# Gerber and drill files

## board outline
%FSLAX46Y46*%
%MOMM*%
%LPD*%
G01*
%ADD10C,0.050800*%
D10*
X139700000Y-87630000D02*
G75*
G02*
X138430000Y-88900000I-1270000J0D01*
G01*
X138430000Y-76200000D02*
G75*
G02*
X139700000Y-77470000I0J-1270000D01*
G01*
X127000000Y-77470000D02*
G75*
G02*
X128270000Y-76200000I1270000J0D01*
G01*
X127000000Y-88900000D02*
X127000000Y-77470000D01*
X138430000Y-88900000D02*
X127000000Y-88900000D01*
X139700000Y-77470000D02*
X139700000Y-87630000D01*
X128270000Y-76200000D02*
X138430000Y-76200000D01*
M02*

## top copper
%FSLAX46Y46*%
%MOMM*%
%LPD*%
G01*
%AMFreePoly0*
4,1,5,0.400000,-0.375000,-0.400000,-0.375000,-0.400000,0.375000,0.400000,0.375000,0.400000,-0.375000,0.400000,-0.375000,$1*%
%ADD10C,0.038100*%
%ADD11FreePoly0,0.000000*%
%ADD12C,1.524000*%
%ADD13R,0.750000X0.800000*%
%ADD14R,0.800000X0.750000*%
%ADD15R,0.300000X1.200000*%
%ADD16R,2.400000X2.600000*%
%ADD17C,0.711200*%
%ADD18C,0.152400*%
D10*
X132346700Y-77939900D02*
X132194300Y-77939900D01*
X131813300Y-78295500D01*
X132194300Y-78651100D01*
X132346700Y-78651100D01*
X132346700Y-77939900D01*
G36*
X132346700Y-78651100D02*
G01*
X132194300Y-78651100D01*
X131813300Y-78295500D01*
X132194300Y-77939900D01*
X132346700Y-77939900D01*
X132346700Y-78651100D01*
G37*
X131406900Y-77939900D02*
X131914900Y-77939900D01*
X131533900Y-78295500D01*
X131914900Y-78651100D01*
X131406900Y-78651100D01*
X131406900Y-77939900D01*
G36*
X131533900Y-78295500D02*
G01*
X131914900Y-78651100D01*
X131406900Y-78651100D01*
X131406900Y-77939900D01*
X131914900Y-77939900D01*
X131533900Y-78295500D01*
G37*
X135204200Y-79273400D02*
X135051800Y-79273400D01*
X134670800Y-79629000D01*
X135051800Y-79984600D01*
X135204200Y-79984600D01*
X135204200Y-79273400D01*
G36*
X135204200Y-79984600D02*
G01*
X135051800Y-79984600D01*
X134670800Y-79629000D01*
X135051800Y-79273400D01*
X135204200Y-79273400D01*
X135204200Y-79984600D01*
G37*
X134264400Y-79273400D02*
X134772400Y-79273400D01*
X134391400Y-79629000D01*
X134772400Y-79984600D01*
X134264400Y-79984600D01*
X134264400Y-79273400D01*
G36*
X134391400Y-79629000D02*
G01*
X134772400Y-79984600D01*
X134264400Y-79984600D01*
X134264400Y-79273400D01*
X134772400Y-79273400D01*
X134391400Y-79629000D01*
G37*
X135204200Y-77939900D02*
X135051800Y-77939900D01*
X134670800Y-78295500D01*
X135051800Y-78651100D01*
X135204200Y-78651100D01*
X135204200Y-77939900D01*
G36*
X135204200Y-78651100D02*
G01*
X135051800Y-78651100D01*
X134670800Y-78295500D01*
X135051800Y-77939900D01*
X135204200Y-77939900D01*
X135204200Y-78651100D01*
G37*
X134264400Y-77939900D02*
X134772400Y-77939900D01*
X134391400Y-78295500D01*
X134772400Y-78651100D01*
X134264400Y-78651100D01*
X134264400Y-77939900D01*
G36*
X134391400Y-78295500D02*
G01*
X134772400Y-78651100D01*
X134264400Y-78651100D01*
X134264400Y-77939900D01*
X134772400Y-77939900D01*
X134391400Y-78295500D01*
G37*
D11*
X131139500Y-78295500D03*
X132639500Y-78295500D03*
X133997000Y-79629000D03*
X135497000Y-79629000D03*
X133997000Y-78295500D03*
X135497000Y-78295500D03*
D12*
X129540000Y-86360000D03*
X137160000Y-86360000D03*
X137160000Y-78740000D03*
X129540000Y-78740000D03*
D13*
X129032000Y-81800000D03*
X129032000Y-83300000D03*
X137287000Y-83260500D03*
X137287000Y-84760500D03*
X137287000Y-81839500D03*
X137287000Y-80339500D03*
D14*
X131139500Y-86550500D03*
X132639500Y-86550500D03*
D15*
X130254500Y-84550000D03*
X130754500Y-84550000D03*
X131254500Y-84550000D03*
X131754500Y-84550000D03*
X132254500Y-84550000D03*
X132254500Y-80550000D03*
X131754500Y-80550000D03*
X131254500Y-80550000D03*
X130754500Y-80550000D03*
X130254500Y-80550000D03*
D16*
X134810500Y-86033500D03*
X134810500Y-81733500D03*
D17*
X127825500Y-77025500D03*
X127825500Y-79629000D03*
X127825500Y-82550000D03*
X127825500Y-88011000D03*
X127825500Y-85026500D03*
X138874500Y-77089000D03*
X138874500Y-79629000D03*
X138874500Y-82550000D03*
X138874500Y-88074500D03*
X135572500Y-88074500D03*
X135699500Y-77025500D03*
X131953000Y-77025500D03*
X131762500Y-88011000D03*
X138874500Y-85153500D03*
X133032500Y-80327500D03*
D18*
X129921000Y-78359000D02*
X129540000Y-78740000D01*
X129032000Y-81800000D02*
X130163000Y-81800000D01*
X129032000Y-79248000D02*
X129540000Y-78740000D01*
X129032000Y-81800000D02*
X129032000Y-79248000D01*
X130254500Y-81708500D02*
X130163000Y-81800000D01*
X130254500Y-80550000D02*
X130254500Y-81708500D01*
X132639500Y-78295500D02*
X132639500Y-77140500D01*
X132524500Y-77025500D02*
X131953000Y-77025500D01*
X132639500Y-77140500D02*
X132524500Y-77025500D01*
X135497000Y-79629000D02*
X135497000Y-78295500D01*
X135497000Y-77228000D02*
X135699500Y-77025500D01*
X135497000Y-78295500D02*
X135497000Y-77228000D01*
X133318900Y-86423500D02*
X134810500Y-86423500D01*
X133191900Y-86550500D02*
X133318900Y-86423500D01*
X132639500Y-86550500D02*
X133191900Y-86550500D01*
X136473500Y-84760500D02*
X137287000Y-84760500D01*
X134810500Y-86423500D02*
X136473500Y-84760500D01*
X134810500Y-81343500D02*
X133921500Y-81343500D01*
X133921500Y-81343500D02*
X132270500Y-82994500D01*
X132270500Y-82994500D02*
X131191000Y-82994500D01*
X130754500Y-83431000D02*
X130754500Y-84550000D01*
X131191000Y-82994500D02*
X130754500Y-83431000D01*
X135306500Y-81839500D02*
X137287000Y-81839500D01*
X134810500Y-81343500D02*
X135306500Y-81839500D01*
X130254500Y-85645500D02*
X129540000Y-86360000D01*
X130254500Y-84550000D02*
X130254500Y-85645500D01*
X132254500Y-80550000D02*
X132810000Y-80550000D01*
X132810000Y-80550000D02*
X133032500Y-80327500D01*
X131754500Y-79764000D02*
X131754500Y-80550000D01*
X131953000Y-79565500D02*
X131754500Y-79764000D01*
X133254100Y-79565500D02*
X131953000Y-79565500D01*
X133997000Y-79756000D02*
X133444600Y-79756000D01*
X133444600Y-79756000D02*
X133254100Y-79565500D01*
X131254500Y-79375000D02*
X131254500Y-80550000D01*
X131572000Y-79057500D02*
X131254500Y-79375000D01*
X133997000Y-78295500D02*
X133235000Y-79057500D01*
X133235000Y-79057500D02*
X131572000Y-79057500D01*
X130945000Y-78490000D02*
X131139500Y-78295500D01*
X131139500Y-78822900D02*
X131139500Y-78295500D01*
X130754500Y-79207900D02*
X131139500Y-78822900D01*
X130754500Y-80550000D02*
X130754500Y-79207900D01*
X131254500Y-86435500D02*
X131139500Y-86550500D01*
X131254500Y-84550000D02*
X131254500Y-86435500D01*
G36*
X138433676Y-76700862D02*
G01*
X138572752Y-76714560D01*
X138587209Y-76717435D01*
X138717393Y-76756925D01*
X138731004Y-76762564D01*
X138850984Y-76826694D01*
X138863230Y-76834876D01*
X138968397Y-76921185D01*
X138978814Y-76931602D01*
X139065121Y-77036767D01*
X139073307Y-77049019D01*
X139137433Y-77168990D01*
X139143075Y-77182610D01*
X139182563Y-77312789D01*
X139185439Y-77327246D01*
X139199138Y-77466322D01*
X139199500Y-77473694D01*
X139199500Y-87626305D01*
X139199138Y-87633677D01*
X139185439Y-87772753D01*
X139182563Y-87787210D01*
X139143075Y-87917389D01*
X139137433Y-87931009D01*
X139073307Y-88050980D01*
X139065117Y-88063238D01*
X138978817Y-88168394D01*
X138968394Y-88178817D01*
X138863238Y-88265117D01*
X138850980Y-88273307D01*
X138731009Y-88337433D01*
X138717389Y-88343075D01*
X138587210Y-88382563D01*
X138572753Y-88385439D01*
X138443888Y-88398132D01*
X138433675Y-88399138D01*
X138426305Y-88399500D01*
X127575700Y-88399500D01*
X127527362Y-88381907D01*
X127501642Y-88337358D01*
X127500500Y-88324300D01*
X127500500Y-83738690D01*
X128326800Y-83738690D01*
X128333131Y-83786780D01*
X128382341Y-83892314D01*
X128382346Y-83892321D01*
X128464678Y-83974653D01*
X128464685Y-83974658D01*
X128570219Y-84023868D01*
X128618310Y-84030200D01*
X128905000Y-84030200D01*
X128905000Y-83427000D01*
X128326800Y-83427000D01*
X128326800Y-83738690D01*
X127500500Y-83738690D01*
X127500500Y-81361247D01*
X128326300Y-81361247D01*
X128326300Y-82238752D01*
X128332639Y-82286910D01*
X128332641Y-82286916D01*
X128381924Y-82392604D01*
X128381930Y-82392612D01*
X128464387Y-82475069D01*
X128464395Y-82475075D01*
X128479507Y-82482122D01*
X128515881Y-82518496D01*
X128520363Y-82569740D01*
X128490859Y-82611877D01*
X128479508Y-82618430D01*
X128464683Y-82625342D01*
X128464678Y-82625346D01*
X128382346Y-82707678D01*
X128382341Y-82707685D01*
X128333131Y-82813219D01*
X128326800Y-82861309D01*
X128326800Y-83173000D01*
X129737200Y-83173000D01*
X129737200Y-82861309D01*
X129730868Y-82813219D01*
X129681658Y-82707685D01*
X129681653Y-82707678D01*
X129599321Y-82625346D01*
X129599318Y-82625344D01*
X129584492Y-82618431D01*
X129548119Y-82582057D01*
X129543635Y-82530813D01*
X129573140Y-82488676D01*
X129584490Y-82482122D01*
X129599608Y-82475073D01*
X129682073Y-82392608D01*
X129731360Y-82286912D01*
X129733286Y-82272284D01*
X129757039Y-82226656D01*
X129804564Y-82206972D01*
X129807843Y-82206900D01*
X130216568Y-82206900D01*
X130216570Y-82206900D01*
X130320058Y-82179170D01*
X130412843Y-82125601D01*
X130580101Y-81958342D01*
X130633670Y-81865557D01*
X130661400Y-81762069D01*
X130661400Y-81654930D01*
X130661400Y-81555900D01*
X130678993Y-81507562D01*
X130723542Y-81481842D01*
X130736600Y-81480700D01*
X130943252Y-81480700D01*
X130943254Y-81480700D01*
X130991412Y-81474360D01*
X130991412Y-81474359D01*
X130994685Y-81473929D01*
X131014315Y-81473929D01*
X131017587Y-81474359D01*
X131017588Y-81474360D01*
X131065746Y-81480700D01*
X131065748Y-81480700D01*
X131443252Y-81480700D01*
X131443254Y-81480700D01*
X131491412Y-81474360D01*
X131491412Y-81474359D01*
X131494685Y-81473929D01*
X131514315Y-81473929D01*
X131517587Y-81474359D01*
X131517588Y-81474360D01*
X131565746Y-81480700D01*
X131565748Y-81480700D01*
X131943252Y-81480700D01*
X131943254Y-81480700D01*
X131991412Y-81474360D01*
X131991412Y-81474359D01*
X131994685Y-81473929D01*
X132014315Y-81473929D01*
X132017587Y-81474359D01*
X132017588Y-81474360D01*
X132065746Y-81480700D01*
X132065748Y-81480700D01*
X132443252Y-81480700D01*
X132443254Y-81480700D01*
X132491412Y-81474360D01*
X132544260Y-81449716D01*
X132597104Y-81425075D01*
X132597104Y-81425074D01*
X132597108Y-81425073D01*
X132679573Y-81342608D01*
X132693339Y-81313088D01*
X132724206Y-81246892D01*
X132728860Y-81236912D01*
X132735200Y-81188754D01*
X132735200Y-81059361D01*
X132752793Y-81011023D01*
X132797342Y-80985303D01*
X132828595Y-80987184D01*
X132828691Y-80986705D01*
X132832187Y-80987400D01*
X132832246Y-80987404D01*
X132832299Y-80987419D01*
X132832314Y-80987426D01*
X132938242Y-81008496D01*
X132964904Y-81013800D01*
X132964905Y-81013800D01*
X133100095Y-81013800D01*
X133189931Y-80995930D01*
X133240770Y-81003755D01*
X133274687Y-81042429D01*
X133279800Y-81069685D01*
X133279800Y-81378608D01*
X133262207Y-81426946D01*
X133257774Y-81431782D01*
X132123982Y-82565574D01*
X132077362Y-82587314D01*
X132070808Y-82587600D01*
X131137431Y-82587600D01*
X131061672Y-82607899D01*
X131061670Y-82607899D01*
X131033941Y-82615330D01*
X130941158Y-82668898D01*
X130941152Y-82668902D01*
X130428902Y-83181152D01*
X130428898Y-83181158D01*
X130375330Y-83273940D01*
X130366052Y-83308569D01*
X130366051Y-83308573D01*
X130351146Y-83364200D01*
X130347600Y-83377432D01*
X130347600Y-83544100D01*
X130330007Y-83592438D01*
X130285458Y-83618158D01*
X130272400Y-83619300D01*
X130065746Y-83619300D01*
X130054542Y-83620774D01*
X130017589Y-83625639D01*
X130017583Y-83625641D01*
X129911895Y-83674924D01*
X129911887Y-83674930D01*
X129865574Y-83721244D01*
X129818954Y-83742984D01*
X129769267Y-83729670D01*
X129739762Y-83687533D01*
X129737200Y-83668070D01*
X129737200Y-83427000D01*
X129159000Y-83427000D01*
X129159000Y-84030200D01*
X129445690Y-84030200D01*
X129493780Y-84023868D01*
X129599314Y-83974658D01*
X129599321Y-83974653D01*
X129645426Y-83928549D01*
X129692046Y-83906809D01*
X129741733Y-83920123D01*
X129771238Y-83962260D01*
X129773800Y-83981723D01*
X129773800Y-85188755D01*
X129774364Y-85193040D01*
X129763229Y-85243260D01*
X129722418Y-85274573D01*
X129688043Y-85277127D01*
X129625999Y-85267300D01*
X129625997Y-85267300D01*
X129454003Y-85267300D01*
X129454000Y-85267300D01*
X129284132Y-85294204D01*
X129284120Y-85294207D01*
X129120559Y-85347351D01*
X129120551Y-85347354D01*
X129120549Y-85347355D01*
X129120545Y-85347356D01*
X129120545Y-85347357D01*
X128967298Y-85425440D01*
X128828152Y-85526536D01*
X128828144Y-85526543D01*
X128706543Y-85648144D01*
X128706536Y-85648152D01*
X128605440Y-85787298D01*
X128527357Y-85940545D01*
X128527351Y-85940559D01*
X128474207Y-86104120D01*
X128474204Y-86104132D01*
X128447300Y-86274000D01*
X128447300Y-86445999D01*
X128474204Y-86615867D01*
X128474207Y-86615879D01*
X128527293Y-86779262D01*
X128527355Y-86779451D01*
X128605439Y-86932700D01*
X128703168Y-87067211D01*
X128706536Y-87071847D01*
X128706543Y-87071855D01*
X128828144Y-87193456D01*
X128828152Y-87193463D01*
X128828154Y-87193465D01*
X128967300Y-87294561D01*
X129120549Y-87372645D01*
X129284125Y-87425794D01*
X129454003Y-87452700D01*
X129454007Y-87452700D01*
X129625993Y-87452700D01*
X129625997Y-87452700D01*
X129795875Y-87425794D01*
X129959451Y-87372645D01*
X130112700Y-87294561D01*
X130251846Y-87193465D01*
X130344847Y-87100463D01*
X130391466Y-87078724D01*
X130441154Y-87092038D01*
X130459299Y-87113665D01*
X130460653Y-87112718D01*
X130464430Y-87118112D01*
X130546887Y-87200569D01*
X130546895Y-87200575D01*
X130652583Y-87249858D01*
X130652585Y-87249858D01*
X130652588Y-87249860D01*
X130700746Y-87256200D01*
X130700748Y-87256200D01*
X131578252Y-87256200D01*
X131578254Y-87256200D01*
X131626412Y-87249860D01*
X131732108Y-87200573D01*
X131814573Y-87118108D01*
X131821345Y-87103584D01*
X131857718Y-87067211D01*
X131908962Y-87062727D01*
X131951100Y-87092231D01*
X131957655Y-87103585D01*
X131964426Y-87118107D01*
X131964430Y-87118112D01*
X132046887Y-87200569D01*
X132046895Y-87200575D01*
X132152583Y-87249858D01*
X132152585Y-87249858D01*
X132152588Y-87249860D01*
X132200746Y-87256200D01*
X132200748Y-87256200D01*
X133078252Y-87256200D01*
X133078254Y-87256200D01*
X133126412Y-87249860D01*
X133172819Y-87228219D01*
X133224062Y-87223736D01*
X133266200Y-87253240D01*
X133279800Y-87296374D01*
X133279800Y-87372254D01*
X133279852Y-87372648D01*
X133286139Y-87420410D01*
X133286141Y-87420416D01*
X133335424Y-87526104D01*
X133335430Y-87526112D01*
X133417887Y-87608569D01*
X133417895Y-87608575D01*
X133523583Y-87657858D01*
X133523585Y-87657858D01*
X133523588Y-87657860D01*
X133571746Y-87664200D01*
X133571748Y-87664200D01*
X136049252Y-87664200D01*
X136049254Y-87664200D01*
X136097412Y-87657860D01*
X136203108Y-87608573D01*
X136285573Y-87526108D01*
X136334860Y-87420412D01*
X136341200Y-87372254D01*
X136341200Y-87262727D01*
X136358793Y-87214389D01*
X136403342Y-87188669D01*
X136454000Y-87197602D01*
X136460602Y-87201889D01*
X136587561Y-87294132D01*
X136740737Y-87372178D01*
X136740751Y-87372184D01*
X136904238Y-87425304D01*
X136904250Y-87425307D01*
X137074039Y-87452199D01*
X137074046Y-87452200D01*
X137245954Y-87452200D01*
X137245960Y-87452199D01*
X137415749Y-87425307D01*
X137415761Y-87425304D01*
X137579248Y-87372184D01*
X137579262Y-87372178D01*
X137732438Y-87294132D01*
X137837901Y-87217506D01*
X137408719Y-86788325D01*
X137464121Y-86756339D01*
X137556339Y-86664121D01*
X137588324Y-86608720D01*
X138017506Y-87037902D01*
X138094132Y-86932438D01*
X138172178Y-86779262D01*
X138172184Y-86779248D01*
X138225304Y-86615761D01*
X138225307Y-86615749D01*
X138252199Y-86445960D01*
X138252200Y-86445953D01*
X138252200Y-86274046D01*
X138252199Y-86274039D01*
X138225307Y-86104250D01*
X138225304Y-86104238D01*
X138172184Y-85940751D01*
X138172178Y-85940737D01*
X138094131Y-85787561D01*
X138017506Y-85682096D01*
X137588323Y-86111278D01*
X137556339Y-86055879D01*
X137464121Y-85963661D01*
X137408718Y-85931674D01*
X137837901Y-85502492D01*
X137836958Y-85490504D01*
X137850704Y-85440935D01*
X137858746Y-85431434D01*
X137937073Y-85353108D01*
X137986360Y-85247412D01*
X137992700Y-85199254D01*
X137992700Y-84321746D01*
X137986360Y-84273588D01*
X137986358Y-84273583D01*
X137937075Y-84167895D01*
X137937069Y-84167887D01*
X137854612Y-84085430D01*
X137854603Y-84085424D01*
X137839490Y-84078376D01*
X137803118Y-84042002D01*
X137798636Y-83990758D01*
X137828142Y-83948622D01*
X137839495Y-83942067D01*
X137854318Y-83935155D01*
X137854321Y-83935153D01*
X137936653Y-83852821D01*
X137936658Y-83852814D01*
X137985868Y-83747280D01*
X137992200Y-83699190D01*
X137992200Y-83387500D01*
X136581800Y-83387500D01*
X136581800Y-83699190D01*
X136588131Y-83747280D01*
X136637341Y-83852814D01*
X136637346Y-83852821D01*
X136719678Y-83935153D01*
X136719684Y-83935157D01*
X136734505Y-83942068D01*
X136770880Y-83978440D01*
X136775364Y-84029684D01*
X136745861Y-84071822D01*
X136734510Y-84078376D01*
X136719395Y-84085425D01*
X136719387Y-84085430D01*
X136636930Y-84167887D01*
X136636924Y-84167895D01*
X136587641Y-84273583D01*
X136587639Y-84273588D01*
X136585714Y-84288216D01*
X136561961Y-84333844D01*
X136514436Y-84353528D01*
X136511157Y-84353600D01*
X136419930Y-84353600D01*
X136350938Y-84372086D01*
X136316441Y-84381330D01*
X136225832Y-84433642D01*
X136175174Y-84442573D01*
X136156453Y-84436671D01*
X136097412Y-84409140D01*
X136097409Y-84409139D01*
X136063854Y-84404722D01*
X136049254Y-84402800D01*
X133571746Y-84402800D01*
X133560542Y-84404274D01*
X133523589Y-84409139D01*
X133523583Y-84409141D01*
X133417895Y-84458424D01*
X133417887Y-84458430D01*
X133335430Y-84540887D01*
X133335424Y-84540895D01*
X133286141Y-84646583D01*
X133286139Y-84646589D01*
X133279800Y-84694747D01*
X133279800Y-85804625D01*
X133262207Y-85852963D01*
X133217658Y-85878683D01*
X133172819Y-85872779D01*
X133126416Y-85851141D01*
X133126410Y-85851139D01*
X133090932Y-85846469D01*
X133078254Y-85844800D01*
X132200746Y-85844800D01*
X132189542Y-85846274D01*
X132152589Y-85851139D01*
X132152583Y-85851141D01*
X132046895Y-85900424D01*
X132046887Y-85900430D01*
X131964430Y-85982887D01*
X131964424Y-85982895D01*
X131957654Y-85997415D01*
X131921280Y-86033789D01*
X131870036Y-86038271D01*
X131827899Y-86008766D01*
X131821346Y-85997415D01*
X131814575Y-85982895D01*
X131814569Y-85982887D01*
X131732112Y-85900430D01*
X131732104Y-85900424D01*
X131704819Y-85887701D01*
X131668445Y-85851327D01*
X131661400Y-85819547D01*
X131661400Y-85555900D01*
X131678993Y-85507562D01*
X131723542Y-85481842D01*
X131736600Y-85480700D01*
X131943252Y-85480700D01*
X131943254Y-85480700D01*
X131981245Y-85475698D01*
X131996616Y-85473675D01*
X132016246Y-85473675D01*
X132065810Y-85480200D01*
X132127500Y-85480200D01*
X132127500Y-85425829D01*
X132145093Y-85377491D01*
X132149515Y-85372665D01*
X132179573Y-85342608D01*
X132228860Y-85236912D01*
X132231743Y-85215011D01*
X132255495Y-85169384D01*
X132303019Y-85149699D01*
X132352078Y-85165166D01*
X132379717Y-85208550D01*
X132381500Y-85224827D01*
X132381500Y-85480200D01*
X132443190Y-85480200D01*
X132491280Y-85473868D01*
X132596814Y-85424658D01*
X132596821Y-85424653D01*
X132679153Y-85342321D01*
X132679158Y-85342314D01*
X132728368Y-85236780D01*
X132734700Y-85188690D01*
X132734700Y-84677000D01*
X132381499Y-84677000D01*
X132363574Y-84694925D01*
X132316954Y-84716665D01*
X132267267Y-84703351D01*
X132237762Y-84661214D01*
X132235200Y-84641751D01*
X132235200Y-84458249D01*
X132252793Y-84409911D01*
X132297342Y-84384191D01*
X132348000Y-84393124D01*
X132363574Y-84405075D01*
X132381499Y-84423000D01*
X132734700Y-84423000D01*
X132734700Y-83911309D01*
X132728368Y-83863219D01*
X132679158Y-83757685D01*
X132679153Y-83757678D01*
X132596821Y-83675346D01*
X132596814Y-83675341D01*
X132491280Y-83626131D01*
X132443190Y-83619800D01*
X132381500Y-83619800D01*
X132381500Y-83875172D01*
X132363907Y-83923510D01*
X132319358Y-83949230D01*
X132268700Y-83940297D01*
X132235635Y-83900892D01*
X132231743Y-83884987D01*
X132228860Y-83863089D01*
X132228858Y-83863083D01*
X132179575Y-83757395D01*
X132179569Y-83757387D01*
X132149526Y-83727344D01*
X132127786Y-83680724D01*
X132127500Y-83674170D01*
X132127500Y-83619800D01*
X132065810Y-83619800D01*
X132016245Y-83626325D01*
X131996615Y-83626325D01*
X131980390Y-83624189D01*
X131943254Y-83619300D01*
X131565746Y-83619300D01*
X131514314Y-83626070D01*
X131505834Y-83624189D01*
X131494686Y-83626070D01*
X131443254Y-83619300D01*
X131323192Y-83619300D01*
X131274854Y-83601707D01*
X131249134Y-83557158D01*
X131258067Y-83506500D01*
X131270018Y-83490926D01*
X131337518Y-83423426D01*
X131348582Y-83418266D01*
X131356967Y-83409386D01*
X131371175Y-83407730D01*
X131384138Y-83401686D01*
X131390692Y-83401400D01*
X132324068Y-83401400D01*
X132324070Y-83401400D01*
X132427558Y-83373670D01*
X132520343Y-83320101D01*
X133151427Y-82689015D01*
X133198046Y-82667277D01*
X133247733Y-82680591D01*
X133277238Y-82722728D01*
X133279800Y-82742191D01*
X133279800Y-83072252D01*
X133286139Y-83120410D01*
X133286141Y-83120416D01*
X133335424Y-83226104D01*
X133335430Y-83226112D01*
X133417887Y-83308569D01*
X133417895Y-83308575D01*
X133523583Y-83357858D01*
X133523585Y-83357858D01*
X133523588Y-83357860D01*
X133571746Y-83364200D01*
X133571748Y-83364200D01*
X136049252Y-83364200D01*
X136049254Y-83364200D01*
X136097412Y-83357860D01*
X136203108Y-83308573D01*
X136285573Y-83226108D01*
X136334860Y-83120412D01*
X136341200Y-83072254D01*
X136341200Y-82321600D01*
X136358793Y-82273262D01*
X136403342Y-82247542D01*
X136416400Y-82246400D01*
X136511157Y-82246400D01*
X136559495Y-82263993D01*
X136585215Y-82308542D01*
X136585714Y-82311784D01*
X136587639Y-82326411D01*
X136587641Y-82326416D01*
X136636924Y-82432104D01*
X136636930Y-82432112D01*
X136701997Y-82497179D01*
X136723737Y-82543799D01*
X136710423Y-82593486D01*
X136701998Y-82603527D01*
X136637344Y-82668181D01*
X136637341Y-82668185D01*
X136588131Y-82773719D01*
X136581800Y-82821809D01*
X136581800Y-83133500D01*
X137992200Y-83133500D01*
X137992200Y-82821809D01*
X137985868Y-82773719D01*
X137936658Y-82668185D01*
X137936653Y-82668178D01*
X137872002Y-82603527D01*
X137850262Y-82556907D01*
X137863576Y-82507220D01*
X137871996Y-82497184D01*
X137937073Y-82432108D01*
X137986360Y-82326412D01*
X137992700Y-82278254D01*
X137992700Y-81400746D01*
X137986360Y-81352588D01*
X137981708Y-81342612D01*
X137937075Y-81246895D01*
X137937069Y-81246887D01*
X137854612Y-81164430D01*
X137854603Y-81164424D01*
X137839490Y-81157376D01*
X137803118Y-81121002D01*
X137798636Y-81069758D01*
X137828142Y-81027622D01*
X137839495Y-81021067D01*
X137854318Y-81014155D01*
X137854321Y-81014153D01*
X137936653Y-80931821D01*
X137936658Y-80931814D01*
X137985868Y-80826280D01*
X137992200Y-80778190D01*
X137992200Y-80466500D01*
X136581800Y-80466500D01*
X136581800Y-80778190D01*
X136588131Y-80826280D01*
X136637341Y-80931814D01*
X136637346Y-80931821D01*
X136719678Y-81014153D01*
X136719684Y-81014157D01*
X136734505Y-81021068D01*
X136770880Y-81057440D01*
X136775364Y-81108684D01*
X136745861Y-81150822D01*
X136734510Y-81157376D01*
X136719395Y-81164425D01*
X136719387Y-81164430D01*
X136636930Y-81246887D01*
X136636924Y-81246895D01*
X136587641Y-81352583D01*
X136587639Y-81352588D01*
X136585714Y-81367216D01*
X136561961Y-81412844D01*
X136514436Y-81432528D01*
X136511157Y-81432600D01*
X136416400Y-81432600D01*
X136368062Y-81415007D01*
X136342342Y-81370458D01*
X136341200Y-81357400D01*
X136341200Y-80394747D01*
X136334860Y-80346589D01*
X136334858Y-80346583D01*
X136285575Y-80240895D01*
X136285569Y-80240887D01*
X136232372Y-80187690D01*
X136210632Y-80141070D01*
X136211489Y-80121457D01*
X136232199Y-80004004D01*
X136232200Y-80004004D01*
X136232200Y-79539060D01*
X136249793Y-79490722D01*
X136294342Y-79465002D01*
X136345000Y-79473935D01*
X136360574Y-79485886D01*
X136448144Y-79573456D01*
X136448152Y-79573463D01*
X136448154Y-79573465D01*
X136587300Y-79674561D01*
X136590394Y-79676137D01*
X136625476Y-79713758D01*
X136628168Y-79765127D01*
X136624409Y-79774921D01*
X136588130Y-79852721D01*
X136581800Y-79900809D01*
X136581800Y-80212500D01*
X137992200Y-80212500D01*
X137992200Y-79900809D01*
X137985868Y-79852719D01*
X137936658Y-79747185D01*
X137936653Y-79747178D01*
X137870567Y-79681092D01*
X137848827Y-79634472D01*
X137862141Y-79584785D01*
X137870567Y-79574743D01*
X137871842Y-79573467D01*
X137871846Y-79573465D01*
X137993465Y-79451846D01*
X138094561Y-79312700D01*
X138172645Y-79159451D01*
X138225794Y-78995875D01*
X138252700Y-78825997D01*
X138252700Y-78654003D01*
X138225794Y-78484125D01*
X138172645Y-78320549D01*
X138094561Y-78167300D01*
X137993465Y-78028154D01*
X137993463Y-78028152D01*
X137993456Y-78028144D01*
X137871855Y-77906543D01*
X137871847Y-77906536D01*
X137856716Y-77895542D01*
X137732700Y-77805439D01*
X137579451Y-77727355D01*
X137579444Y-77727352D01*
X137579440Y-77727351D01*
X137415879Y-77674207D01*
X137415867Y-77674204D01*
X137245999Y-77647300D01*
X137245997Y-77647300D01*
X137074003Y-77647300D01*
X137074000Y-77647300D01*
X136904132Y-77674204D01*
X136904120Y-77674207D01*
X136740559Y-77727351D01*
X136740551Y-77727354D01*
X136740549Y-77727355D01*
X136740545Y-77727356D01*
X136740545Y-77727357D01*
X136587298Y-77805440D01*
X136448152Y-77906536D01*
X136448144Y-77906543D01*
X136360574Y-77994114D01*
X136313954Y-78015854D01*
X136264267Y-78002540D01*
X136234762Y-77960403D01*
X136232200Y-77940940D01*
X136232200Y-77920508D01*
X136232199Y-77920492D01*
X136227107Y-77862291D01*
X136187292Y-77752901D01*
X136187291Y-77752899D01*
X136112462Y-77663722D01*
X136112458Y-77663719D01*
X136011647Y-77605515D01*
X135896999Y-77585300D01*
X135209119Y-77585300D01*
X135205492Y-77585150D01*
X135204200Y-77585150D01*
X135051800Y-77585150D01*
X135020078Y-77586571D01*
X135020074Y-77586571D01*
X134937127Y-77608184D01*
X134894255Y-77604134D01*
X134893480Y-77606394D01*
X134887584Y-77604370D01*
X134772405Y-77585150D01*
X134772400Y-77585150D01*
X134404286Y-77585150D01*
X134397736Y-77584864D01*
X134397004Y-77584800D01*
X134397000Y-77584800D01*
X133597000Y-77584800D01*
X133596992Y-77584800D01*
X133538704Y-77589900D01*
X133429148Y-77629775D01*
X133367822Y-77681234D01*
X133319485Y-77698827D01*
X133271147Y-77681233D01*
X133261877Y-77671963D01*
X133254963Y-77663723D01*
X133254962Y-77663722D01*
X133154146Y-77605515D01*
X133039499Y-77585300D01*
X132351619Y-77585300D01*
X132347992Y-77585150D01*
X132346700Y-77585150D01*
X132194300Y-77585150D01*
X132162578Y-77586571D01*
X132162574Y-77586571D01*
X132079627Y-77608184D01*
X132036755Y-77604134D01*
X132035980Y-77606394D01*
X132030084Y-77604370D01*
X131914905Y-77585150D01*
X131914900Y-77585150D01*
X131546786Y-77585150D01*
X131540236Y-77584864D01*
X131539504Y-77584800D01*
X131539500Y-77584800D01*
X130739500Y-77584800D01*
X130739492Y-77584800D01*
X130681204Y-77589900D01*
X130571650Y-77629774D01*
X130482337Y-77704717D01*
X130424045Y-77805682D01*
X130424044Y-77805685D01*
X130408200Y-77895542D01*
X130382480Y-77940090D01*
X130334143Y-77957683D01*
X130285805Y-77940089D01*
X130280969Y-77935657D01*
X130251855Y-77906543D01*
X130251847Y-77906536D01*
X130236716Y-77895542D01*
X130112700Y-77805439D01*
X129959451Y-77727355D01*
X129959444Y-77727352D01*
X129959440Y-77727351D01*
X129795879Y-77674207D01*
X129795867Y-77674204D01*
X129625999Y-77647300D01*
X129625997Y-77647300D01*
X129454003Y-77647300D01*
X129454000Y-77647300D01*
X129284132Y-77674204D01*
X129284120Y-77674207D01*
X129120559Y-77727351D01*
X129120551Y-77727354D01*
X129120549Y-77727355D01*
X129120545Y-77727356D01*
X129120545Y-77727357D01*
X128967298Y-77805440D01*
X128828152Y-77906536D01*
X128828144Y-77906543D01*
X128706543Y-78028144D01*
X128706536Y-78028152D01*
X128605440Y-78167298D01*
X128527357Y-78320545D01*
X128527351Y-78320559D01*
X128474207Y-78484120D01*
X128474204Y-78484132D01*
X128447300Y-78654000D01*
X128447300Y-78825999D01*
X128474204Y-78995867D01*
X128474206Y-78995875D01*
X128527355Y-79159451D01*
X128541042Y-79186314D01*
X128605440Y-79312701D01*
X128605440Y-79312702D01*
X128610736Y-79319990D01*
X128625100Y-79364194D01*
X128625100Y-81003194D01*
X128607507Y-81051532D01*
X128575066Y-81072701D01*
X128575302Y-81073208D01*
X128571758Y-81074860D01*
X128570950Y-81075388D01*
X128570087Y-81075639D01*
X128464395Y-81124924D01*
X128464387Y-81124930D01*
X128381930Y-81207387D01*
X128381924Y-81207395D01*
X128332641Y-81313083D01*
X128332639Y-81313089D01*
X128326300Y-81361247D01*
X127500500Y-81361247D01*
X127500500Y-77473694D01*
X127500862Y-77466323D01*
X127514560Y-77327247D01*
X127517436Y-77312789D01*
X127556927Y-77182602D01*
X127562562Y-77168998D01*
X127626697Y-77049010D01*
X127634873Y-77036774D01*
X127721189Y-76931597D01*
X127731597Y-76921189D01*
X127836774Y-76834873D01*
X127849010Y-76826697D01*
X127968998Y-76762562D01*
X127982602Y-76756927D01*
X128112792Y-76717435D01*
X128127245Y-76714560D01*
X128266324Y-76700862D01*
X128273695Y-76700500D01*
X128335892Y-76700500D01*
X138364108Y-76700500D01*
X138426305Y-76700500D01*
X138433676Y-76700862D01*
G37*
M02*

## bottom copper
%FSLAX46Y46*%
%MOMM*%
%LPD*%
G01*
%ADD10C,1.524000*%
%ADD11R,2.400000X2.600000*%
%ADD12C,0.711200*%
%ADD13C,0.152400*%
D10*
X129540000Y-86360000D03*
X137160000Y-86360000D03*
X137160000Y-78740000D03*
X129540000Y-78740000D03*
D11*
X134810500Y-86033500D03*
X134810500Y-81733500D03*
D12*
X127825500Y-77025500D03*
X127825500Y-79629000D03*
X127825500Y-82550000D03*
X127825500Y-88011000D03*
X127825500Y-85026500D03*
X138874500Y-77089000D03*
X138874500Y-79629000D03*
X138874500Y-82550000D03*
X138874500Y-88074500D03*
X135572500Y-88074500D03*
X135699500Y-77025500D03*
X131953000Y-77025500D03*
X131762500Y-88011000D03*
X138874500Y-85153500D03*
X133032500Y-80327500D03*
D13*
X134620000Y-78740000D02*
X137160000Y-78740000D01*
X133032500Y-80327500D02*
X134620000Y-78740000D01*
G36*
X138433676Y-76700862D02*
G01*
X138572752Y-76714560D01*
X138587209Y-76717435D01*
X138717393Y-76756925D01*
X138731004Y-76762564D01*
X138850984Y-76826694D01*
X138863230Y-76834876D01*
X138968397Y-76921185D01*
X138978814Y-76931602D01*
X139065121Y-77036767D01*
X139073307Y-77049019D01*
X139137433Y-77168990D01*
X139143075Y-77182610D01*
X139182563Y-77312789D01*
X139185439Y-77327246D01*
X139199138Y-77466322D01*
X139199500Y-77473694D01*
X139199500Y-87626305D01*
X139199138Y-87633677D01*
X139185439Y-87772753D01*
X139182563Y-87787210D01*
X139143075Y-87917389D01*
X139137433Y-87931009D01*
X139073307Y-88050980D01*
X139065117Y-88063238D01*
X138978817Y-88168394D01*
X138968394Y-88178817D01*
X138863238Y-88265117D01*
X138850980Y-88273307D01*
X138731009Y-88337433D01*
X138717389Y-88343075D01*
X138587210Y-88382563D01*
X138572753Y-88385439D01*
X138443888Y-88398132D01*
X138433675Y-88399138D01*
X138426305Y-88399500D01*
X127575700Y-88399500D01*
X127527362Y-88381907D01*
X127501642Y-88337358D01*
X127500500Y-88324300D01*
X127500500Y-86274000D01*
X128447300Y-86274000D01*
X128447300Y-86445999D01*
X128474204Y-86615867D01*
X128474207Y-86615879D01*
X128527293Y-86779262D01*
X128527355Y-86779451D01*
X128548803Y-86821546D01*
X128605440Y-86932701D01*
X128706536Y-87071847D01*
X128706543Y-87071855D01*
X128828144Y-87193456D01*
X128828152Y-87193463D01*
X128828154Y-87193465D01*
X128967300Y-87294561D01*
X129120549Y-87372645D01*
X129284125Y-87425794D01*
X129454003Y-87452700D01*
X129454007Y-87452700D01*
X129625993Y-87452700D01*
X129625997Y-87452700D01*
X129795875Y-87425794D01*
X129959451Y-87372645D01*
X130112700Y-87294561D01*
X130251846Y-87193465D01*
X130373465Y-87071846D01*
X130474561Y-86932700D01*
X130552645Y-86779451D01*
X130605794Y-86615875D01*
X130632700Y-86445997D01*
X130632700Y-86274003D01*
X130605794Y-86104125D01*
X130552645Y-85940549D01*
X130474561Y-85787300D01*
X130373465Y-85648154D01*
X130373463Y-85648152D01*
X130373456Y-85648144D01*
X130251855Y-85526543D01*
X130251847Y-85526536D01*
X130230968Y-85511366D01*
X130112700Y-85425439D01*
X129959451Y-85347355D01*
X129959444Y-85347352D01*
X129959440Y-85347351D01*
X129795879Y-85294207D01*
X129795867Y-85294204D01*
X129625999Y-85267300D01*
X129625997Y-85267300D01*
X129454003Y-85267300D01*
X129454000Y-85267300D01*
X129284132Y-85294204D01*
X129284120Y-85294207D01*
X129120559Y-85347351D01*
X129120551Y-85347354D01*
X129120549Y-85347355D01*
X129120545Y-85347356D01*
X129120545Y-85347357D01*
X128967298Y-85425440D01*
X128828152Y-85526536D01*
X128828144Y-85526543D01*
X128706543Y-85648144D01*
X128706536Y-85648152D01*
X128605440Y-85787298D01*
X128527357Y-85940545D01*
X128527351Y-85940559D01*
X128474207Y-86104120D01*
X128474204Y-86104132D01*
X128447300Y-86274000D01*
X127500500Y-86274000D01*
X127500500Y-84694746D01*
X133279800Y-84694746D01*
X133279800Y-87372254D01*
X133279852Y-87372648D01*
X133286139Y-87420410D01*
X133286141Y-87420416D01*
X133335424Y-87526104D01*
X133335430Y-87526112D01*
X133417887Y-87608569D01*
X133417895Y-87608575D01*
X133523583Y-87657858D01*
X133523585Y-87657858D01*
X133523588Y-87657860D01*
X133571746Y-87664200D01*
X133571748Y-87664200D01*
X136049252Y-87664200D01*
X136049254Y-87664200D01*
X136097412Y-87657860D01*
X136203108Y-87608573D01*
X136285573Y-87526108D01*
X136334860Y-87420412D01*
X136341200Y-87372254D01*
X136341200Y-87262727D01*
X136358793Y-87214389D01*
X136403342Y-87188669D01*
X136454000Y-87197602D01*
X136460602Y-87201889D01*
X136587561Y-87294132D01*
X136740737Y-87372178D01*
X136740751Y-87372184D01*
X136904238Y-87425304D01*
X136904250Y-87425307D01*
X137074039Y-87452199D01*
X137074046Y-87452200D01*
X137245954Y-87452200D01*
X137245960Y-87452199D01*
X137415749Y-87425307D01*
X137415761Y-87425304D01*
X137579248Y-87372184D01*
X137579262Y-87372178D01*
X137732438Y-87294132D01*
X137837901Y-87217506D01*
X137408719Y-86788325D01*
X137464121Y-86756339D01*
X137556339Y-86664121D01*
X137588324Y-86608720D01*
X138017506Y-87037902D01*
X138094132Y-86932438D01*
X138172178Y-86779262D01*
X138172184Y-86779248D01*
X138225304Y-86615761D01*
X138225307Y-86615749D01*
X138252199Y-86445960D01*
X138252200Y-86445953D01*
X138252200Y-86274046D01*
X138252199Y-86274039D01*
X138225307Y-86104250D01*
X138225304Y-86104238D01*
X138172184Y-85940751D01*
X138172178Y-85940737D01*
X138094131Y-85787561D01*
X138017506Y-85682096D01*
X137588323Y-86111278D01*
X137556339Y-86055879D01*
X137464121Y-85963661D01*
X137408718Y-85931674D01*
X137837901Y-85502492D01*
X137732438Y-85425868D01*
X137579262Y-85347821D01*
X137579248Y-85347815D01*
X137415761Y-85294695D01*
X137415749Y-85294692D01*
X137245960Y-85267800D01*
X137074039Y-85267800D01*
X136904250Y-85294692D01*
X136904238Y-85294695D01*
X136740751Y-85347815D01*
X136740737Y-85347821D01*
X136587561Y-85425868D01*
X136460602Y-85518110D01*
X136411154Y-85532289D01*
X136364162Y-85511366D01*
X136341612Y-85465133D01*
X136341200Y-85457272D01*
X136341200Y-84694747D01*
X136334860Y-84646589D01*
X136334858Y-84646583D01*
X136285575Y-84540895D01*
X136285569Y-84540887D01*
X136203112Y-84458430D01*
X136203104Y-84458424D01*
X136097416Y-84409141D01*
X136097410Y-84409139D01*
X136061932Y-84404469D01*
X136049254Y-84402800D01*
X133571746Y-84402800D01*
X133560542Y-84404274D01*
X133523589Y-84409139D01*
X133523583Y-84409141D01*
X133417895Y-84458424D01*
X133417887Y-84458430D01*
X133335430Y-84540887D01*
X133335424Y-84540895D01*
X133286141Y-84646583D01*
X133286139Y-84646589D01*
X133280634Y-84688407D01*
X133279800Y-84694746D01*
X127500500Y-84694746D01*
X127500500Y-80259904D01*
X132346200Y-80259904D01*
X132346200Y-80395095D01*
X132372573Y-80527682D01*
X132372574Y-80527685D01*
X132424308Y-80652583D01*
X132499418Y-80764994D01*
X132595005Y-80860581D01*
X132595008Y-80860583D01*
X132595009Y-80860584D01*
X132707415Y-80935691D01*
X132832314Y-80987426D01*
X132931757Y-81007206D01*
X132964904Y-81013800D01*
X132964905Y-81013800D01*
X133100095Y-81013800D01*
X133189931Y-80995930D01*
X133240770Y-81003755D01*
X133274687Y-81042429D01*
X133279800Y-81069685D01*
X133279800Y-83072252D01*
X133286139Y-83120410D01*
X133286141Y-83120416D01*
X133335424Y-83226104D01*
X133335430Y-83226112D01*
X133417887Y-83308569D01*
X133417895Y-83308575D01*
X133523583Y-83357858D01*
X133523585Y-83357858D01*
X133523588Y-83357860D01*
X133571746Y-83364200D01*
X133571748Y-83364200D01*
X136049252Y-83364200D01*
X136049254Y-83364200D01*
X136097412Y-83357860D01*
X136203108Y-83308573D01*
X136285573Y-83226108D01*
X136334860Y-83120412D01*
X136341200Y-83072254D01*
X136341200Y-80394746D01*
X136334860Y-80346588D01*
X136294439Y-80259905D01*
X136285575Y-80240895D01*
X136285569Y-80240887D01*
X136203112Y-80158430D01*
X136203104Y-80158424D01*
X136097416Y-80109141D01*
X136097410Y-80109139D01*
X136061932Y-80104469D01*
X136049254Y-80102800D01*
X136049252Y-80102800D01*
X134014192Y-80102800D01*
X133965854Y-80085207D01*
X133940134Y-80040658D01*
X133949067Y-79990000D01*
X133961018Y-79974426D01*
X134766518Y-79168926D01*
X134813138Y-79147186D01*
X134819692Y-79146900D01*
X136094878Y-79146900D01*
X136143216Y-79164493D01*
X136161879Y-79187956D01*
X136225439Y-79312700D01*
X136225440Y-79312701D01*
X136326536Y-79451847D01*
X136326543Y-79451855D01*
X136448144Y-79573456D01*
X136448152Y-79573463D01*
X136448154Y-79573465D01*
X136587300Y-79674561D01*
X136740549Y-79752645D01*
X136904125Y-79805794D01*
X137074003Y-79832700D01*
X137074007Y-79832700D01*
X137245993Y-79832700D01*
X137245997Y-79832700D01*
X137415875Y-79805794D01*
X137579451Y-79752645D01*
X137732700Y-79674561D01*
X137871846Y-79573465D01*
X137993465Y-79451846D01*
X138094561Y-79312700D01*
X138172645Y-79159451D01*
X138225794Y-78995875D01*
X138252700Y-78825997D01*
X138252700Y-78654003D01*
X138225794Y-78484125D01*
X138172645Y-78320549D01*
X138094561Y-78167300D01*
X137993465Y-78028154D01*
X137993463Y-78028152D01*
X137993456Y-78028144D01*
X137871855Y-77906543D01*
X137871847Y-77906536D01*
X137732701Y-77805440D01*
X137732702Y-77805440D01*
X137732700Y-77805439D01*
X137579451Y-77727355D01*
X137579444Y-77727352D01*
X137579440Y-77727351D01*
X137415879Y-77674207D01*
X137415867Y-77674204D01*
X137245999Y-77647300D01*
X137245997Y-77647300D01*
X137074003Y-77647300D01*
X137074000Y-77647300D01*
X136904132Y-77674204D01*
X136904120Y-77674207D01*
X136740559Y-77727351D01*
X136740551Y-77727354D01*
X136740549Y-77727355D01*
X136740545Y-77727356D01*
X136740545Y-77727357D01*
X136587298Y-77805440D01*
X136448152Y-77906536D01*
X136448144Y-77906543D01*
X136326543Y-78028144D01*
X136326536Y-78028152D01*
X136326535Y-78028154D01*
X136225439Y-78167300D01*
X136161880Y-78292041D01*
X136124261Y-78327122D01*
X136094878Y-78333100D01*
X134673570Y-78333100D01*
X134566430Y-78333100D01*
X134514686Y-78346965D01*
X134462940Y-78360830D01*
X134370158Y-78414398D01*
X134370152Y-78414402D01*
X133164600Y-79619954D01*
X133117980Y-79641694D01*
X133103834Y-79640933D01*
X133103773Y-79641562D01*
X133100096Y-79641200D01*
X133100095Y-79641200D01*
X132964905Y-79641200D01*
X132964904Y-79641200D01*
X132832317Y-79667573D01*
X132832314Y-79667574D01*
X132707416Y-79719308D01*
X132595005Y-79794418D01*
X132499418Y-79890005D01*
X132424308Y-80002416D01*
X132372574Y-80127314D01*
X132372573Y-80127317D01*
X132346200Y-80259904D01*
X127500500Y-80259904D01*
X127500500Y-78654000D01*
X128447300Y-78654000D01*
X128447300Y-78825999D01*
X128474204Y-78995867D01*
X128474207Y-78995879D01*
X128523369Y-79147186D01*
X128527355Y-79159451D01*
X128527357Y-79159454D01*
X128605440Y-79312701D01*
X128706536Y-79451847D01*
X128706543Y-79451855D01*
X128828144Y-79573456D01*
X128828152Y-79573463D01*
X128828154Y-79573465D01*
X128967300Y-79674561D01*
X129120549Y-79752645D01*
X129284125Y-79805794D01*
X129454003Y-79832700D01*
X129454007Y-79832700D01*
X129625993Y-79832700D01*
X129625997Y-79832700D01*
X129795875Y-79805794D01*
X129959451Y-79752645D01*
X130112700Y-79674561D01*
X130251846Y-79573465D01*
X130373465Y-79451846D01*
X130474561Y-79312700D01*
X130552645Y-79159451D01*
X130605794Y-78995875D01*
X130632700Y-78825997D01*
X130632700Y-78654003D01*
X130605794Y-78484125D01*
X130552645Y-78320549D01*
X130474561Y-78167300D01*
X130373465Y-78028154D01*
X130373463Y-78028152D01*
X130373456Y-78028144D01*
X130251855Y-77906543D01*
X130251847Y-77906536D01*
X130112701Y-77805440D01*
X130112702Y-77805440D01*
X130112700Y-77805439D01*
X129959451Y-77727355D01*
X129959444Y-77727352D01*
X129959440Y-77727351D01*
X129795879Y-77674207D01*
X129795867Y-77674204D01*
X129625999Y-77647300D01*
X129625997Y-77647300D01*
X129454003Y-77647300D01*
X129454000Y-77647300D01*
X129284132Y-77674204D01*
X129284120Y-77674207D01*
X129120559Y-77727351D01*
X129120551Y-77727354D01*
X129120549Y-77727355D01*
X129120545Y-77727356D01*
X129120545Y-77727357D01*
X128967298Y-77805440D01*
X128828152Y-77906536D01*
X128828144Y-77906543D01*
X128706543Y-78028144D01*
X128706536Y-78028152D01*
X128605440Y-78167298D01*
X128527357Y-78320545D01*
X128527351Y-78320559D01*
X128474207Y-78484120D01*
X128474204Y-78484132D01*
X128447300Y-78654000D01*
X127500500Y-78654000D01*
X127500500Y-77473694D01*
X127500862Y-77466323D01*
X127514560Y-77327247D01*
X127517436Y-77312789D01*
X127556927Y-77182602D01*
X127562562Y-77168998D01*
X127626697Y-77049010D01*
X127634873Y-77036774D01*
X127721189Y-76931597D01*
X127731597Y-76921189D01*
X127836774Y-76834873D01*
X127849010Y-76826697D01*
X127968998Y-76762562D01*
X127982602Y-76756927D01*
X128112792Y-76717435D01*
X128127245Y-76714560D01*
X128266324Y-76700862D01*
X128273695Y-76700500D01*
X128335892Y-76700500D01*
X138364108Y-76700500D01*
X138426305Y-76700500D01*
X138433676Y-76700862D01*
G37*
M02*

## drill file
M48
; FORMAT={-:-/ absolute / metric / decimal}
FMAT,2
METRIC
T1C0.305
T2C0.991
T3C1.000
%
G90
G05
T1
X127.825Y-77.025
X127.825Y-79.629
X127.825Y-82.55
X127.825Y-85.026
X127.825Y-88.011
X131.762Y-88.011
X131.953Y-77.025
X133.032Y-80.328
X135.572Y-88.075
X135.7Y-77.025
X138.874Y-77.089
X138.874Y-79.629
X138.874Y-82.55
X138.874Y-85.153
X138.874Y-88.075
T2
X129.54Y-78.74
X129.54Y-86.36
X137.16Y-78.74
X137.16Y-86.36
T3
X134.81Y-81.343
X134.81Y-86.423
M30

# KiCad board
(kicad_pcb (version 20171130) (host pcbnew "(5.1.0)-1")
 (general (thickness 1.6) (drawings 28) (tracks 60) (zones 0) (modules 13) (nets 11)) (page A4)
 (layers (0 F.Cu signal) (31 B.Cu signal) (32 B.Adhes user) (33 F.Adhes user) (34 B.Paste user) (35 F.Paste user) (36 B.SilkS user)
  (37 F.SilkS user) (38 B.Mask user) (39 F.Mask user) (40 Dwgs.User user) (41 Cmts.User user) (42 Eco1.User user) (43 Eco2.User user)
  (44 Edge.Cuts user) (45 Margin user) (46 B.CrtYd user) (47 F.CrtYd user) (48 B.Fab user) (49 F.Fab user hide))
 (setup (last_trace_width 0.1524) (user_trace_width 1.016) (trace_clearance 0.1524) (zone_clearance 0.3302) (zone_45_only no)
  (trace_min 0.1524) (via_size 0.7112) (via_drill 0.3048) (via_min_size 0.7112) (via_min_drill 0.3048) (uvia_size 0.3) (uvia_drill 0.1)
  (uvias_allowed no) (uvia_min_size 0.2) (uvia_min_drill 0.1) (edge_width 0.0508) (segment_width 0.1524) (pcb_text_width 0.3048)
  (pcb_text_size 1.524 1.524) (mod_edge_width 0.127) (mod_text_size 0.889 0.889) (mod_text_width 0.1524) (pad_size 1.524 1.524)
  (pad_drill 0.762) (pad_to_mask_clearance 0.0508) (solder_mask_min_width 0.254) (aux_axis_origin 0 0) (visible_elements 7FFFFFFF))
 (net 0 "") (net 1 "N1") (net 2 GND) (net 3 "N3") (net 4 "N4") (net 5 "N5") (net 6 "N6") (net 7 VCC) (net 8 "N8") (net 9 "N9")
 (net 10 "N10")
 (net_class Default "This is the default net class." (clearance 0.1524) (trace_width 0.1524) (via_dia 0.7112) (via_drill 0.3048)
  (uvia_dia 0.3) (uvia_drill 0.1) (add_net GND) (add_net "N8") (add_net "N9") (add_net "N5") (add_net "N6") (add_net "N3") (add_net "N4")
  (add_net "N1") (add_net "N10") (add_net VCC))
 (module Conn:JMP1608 (layer F.Cu) (at 131.8895 78.2955)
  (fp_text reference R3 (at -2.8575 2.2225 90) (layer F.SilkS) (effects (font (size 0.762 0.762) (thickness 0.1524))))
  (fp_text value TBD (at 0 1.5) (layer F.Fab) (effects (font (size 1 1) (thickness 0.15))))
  (fp_poly (pts (xy 0.4572 -0.3556) (xy 0.3048 -0.3556) (xy -0.0762 0) (xy 0.3048 0.3556) (xy 0.4572 0.3556)) (layer F.Cu) (width 0.0381))
  (fp_poly (pts (xy -0.4826 -0.3556) (xy 0.0254 -0.3556) (xy -0.3556 0) (xy 0.0254 0.3556) (xy -0.4826 0.3556)) (layer F.Cu) (width 0.0381))
  (pad 1 smd custom (at -0.75 0) (size 0.8 0.75) (layers F.Cu F.Mask) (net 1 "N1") (zone_connect 0)
   (options (clearance outline) (anchor rect)) (primitives))
  (pad 2 smd custom (at 0.75 0) (size 0.8 0.75) (layers F.Cu F.Mask) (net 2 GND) (zone_connect 0)
   (options (clearance outline) (anchor rect)) (primitives)))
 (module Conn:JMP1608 (layer F.Cu) (at 134.747 79.629)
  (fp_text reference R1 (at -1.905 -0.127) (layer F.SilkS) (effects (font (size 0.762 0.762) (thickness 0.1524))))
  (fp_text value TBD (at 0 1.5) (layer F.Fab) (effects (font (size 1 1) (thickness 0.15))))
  (fp_poly (pts (xy 0.4572 -0.3556) (xy 0.3048 -0.3556) (xy -0.0762 0) (xy 0.3048 0.3556) (xy 0.4572 0.3556)) (layer F.Cu) (width 0.0381))
  (fp_poly (pts (xy -0.4826 -0.3556) (xy 0.0254 -0.3556) (xy -0.3556 0) (xy 0.0254 0.3556) (xy -0.4826 0.3556)) (layer F.Cu) (width 0.0381))
  (pad 1 smd custom (at -0.75 0) (size 0.8 0.75) (layers F.Cu F.Mask) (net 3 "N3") (zone_connect 0)
   (options (clearance outline) (anchor rect)) (primitives))
  (pad 2 smd custom (at 0.75 0) (size 0.8 0.75) (layers F.Cu F.Mask) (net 2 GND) (zone_connect 0)
   (options (clearance outline) (anchor rect)) (primitives)))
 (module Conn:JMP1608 (layer F.Cu) (at 134.747 78.2955)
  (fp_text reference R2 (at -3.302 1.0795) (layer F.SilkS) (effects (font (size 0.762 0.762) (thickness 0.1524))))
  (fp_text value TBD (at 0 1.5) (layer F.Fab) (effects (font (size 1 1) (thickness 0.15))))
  (fp_poly (pts (xy 0.4572 -0.3556) (xy 0.3048 -0.3556) (xy -0.0762 0) (xy 0.3048 0.3556) (xy 0.4572 0.3556)) (layer F.Cu) (width 0.0381))
  (fp_poly (pts (xy -0.4826 -0.3556) (xy 0.0254 -0.3556) (xy -0.3556 0) (xy 0.0254 0.3556) (xy -0.4826 0.3556)) (layer F.Cu) (width 0.0381))
  (pad 1 smd custom (at -0.75 0) (size 0.8 0.75) (layers F.Cu F.Mask) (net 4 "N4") (zone_connect 0)
   (options (clearance outline) (anchor rect)) (primitives))
  (pad 2 smd custom (at 0.75 0) (size 0.8 0.75) (layers F.Cu F.Mask) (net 2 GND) (zone_connect 0)
   (options (clearance outline) (anchor rect)) (primitives)))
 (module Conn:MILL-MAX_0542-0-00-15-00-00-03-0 (layer F.Cu) (at 129.54 86.36)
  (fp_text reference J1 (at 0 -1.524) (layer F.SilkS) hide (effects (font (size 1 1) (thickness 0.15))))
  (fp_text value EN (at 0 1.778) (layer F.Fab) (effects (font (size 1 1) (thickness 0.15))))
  (pad 1 thru_hole circle (at 0 0) (size 1.524 1.524) (drill 0.9906) (layers *.Cu *.Mask) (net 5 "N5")))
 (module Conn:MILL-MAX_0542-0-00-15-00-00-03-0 (layer F.Cu) (at 137.16 86.36)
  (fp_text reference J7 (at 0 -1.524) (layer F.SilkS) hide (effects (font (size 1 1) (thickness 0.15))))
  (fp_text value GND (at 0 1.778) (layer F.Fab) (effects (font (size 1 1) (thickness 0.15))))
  (pad 1 thru_hole circle (at 0 0) (size 1.524 1.524) (drill 0.9906) (layers *.Cu *.Mask) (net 2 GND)))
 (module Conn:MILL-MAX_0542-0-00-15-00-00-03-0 (layer F.Cu) (at 137.16 78.74)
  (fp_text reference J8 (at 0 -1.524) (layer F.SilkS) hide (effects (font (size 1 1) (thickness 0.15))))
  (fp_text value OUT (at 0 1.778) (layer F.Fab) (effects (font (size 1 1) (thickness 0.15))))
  (pad 1 thru_hole circle (at 0 0) (size 1.524 1.524) (drill 0.9906) (layers *.Cu *.Mask) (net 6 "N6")))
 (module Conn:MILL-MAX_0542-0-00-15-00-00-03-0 (layer F.Cu) (at 129.54 78.74)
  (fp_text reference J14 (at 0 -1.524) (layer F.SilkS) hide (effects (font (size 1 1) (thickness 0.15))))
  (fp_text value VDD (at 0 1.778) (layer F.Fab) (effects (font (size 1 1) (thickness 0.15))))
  (pad 1 thru_hole circle (at 0 0) (size 1.524 1.524) (drill 0.9906) (layers *.Cu *.Mask) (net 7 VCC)))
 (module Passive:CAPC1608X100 (layer F.Cu) (at 129.032 82.55 270)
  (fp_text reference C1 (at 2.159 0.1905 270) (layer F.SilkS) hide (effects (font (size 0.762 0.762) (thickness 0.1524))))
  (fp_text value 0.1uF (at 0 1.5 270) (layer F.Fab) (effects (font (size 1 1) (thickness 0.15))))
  (pad 1 smd rect (at -0.75 0 270) (size 0.8 0.75) (layers F.Cu F.Paste F.Mask) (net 7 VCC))
  (pad 2 smd rect (at 0.75 0 270) (size 0.8 0.75) (layers F.Cu F.Paste F.Mask) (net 2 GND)))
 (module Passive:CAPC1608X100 (layer F.Cu) (at 137.287 84.0105 90)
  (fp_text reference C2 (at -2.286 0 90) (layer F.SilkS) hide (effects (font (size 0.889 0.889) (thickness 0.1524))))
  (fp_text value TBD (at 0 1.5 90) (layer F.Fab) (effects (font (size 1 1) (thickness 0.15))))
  (pad 2 smd rect (at 0.75 0 90) (size 0.8 0.75) (layers F.Cu F.Paste F.Mask) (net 2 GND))
  (pad 1 smd rect (at -0.75 0 90) (size 0.8 0.75) (layers F.Cu F.Paste F.Mask) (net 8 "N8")))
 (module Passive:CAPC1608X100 (layer F.Cu) (at 137.287 81.0895 90)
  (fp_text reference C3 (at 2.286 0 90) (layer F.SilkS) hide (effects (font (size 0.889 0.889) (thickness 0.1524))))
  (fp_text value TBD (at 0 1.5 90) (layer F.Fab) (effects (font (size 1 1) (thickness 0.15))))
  (pad 1 smd rect (at -0.75 0 90) (size 0.8 0.75) (layers F.Cu F.Paste F.Mask) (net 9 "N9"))
  (pad 2 smd rect (at 0.75 0 90) (size 0.8 0.75) (layers F.Cu F.Paste F.Mask) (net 2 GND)))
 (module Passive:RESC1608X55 (layer F.Cu) (at 131.8895 86.5505)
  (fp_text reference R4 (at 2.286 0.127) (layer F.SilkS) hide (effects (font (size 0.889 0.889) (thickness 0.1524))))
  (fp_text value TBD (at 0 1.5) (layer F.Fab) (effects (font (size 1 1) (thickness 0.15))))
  (pad 1 smd rect (at -0.75 0) (size 0.8 0.75) (layers F.Cu F.Paste F.Mask) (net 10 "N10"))
  (pad 2 smd rect (at 0.75 0) (size 0.8 0.75) (layers F.Cu F.Paste F.Mask) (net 8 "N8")))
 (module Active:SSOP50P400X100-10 (layer F.Cu) (at 131.2545 82.55 90)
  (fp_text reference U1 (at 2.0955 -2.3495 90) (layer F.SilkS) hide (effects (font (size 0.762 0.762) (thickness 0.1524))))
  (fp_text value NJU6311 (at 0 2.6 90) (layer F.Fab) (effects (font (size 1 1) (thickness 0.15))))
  (pad 1 smd rect (at -2 -1 90) (size 1.2 0.3) (layers F.Cu F.Paste F.Mask) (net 5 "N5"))
  (pad 2 smd rect (at -2 -0.5 90) (size 1.2 0.3) (layers F.Cu F.Paste F.Mask) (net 9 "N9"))
  (pad 3 smd rect (at -2 0 90) (size 1.2 0.3) (layers F.Cu F.Paste F.Mask) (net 10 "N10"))
  (pad 4 smd rect (at -2 0.5 90) (size 1.2 0.3) (layers F.Cu F.Paste F.Mask))
  (pad 5 smd rect (at -2 1 90) (size 1.2 0.3) (layers F.Cu F.Paste F.Mask) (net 2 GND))
  (pad 6 smd rect (at 2 1 90) (size 1.2 0.3) (layers F.Cu F.Paste F.Mask) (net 6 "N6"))
  (pad 7 smd rect (at 2 0.5 90) (size 1.2 0.3) (layers F.Cu F.Paste F.Mask) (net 3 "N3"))
  (pad 8 smd rect (at 2 0 90) (size 1.2 0.3) (layers F.Cu F.Paste F.Mask) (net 4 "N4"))
  (pad 9 smd rect (at 2 -0.5 90) (size 1.2 0.3) (layers F.Cu F.Paste F.Mask) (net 1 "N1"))
  (pad 10 smd rect (at 2 -1 90) (size 1.2 0.3) (layers F.Cu F.Paste F.Mask) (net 7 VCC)))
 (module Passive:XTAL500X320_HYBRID (layer F.Cu) (at 134.8105 83.8835 270)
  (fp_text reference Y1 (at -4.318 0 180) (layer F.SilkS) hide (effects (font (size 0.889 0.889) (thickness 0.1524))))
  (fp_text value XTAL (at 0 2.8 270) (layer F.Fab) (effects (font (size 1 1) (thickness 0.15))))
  (pad 2 thru_hole rect (at 2.54 0 270) (size 2.6 2.4) (drill 1 (offset -0.39 0)) (layers *.Cu *.Mask) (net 8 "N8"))
  (pad 1 thru_hole rect (at -2.54 0 90) (size 2.6 2.4) (drill 1 (offset -0.39 0)) (layers *.Cu *.Mask) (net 9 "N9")))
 (gr_arc (start 138.43 87.63) (end 138.43 88.9) (angle -90) (layer Edge.Cuts) (width 0.0508))
 (gr_arc (start 138.43 77.47) (end 139.7 77.47) (angle -90) (layer Edge.Cuts) (width 0.0508))
 (gr_arc (start 128.27 77.47) (end 128.27 76.2) (angle -90) (layer Edge.Cuts) (width 0.0508))
 (gr_line (start 127 88.9) (end 127 77.47) (layer Edge.Cuts) (width 0.0508))
 (gr_line (start 138.43 88.9) (end 127 88.9) (layer Edge.Cuts) (width 0.0508))
 (gr_line (start 139.7 77.47) (end 139.7 87.63) (layer Edge.Cuts) (width 0.0508))
 (gr_line (start 128.27 76.2) (end 138.43 76.2) (layer Edge.Cuts) (width 0.0508))
 (segment (start 129.921 78.359) (end 129.54 78.74) (width 0.1524) (layer F.Cu) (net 7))
 (segment (start 129.032 81.8) (end 130.163 81.8) (width 0.1524) (layer F.Cu) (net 7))
 (segment (start 129.032 79.248) (end 129.54 78.74) (width 0.1524) (layer F.Cu) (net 7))
 (segment (start 129.032 81.8) (end 129.032 79.248) (width 0.1524) (layer F.Cu) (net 7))
 (segment (start 130.2545 81.7085) (end 130.163 81.8) (width 0.1524) (layer F.Cu) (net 7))
 (segment (start 130.2545 80.55) (end 130.2545 81.7085) (width 0.1524) (layer F.Cu) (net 7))
 (via (at 127.8255 77.0255) (size 0.7112) (drill 0.3048) (layers F.Cu B.Cu) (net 2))
 (via (at 127.8255 79.629) (size 0.7112) (drill 0.3048) (layers F.Cu B.Cu) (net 2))
 (via (at 127.8255 82.55) (size 0.7112) (drill 0.3048) (layers F.Cu B.Cu) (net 2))
 (via (at 127.8255 88.011) (size 0.7112) (drill 0.3048) (layers F.Cu B.Cu) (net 2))
 (via (at 127.8255 85.0265) (size 0.7112) (drill 0.3048) (layers F.Cu B.Cu) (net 2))
 (via (at 138.8745 77.089) (size 0.7112) (drill 0.3048) (layers F.Cu B.Cu) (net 2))
 (via (at 138.8745 79.629) (size 0.7112) (drill 0.3048) (layers F.Cu B.Cu) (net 2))
 (via (at 138.8745 82.55) (size 0.7112) (drill 0.3048) (layers F.Cu B.Cu) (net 2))
 (via (at 138.8745 88.0745) (size 0.7112) (drill 0.3048) (layers F.Cu B.Cu) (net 2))
 (via (at 135.5725 88.0745) (size 0.7112) (drill 0.3048) (layers F.Cu B.Cu) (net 2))
 (via (at 135.6995 77.0255) (size 0.7112) (drill 0.3048) (layers F.Cu B.Cu) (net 2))
 (via (at 131.953 77.0255) (size 0.7112) (drill 0.3048) (layers F.Cu B.Cu) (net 2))
 (via (at 131.7625 88.011) (size 0.7112) (drill 0.3048) (layers F.Cu B.Cu) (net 2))
 (via (at 138.8745 85.1535) (size 0.7112) (drill 0.3048) (layers F.Cu B.Cu) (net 2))
 (segment (start 132.6395 78.2955) (end 132.6395 77.1405) (width 0.1524) (layer F.Cu) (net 2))
 (segment (start 132.5245 77.0255) (end 131.953 77.0255) (width 0.1524) (layer F.Cu) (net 2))
 (segment (start 132.6395 77.1405) (end 132.5245 77.0255) (width 0.1524) (layer F.Cu) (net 2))
 (segment (start 135.497 79.629) (end 135.497 78.2955) (width 0.1524) (layer F.Cu) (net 2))
 (segment (start 135.497 77.228) (end 135.6995 77.0255) (width 0.1524) (layer F.Cu) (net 2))
 (segment (start 135.497 78.2955) (end 135.497 77.228) (width 0.1524) (layer F.Cu) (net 2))
 (segment (start 133.3189 86.4235) (end 134.8105 86.4235) (width 0.1524) (layer F.Cu) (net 8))
 (segment (start 133.1919 86.5505) (end 133.3189 86.4235) (width 0.1524) (layer F.Cu) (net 8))
 (segment (start 132.6395 86.5505) (end 133.1919 86.5505) (width 0.1524) (layer F.Cu) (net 8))
 (segment (start 136.4735 84.7605) (end 137.287 84.7605) (width 0.1524) (layer F.Cu) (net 8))
 (segment (start 134.8105 86.4235) (end 136.4735 84.7605) (width 0.1524) (layer F.Cu) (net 8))
 (segment (start 134.8105 81.3435) (end 133.9215 81.3435) (width 0.1524) (layer F.Cu) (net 9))
 (segment (start 133.9215 81.3435) (end 132.2705 82.9945) (width 0.1524) (layer F.Cu) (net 9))
 (segment (start 132.2705 82.9945) (end 131.191 82.9945) (width 0.1524) (layer F.Cu) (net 9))
 (segment (start 130.7545 83.431) (end 130.7545 84.55) (width 0.1524) (layer F.Cu) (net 9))
 (segment (start 131.191 82.9945) (end 130.7545 83.431) (width 0.1524) (layer F.Cu) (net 9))
 (segment (start 135.3065 81.8395) (end 137.287 81.8395) (width 0.1524) (layer F.Cu) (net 9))
 (segment (start 134.8105 81.3435) (end 135.3065 81.8395) (width 0.1524) (layer F.Cu) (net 9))
 (segment (start 130.2545 85.6455) (end 129.54 86.36) (width 0.1524) (layer F.Cu) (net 5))
 (segment (start 130.2545 84.55) (end 130.2545 85.6455) (width 0.1524) (layer F.Cu) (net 5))
 (via (at 133.0325 80.3275) (size 0.7112) (drill 0.3048) (layers F.Cu B.Cu) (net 6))
 (segment (start 132.2545 80.55) (end 132.81 80.55) (width 0.1524) (layer F.Cu) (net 6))
 (segment (start 132.81 80.55) (end 133.0325 80.3275) (width 0.1524) (layer F.Cu) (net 6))
 (segment (start 134.62 78.74) (end 137.16 78.74) (width 0.1524) (layer B.Cu) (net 6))
 (segment (start 133.0325 80.3275) (end 134.62 78.74) (width 0.1524) (layer B.Cu) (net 6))
 (segment (start 131.7545 79.764) (end 131.7545 80.55) (width 0.1524) (layer F.Cu) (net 3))
 (segment (start 131.953 79.5655) (end 131.7545 79.764) (width 0.1524) (layer F.Cu) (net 3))
 (segment (start 133.2541 79.5655) (end 131.953 79.5655) (width 0.1524) (layer F.Cu) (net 3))
 (segment (start 133.997 79.756) (end 133.4446 79.756) (width 0.1524) (layer F.Cu) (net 3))
 (segment (start 133.4446 79.756) (end 133.2541 79.5655) (width 0.1524) (layer F.Cu) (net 3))
 (segment (start 131.2545 79.375) (end 131.2545 80.55) (width 0.1524) (layer F.Cu) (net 4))
 (segment (start 131.572 79.0575) (end 131.2545 79.375) (width 0.1524) (layer F.Cu) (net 4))
 (segment (start 133.997 78.2955) (end 133.235 79.0575) (width 0.1524) (layer F.Cu) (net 4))
 (segment (start 133.235 79.0575) (end 131.572 79.0575) (width 0.1524) (layer F.Cu) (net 4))
 (segment (start 130.945 78.49) (end 131.1395 78.2955) (width 0.1524) (layer F.Cu) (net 1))
 (segment (start 131.1395 78.8229) (end 131.1395 78.2955) (width 0.1524) (layer F.Cu) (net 1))
 (segment (start 130.7545 79.2079) (end 131.1395 78.8229) (width 0.1524) (layer F.Cu) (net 1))
 (segment (start 130.7545 80.55) (end 130.7545 79.2079) (width 0.1524) (layer F.Cu) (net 1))
 (segment (start 131.2545 86.4355) (end 131.1395 86.5505) (width 0.1524) (layer F.Cu) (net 10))
 (segment (start 131.2545 84.55) (end 131.2545 86.4355) (width 0.1524) (layer F.Cu) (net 10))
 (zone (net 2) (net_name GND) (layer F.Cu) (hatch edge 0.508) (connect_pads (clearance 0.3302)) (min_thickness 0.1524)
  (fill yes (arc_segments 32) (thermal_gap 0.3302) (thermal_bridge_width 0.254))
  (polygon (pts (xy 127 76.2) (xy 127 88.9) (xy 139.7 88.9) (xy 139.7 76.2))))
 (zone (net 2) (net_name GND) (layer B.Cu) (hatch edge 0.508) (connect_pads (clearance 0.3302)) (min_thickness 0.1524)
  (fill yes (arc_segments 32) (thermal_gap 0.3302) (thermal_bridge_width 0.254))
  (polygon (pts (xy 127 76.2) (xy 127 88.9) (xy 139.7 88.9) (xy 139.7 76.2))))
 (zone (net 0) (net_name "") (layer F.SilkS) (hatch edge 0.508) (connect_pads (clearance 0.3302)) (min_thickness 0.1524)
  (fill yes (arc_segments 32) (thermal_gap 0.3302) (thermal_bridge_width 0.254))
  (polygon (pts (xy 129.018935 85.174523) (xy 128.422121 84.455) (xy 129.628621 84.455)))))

